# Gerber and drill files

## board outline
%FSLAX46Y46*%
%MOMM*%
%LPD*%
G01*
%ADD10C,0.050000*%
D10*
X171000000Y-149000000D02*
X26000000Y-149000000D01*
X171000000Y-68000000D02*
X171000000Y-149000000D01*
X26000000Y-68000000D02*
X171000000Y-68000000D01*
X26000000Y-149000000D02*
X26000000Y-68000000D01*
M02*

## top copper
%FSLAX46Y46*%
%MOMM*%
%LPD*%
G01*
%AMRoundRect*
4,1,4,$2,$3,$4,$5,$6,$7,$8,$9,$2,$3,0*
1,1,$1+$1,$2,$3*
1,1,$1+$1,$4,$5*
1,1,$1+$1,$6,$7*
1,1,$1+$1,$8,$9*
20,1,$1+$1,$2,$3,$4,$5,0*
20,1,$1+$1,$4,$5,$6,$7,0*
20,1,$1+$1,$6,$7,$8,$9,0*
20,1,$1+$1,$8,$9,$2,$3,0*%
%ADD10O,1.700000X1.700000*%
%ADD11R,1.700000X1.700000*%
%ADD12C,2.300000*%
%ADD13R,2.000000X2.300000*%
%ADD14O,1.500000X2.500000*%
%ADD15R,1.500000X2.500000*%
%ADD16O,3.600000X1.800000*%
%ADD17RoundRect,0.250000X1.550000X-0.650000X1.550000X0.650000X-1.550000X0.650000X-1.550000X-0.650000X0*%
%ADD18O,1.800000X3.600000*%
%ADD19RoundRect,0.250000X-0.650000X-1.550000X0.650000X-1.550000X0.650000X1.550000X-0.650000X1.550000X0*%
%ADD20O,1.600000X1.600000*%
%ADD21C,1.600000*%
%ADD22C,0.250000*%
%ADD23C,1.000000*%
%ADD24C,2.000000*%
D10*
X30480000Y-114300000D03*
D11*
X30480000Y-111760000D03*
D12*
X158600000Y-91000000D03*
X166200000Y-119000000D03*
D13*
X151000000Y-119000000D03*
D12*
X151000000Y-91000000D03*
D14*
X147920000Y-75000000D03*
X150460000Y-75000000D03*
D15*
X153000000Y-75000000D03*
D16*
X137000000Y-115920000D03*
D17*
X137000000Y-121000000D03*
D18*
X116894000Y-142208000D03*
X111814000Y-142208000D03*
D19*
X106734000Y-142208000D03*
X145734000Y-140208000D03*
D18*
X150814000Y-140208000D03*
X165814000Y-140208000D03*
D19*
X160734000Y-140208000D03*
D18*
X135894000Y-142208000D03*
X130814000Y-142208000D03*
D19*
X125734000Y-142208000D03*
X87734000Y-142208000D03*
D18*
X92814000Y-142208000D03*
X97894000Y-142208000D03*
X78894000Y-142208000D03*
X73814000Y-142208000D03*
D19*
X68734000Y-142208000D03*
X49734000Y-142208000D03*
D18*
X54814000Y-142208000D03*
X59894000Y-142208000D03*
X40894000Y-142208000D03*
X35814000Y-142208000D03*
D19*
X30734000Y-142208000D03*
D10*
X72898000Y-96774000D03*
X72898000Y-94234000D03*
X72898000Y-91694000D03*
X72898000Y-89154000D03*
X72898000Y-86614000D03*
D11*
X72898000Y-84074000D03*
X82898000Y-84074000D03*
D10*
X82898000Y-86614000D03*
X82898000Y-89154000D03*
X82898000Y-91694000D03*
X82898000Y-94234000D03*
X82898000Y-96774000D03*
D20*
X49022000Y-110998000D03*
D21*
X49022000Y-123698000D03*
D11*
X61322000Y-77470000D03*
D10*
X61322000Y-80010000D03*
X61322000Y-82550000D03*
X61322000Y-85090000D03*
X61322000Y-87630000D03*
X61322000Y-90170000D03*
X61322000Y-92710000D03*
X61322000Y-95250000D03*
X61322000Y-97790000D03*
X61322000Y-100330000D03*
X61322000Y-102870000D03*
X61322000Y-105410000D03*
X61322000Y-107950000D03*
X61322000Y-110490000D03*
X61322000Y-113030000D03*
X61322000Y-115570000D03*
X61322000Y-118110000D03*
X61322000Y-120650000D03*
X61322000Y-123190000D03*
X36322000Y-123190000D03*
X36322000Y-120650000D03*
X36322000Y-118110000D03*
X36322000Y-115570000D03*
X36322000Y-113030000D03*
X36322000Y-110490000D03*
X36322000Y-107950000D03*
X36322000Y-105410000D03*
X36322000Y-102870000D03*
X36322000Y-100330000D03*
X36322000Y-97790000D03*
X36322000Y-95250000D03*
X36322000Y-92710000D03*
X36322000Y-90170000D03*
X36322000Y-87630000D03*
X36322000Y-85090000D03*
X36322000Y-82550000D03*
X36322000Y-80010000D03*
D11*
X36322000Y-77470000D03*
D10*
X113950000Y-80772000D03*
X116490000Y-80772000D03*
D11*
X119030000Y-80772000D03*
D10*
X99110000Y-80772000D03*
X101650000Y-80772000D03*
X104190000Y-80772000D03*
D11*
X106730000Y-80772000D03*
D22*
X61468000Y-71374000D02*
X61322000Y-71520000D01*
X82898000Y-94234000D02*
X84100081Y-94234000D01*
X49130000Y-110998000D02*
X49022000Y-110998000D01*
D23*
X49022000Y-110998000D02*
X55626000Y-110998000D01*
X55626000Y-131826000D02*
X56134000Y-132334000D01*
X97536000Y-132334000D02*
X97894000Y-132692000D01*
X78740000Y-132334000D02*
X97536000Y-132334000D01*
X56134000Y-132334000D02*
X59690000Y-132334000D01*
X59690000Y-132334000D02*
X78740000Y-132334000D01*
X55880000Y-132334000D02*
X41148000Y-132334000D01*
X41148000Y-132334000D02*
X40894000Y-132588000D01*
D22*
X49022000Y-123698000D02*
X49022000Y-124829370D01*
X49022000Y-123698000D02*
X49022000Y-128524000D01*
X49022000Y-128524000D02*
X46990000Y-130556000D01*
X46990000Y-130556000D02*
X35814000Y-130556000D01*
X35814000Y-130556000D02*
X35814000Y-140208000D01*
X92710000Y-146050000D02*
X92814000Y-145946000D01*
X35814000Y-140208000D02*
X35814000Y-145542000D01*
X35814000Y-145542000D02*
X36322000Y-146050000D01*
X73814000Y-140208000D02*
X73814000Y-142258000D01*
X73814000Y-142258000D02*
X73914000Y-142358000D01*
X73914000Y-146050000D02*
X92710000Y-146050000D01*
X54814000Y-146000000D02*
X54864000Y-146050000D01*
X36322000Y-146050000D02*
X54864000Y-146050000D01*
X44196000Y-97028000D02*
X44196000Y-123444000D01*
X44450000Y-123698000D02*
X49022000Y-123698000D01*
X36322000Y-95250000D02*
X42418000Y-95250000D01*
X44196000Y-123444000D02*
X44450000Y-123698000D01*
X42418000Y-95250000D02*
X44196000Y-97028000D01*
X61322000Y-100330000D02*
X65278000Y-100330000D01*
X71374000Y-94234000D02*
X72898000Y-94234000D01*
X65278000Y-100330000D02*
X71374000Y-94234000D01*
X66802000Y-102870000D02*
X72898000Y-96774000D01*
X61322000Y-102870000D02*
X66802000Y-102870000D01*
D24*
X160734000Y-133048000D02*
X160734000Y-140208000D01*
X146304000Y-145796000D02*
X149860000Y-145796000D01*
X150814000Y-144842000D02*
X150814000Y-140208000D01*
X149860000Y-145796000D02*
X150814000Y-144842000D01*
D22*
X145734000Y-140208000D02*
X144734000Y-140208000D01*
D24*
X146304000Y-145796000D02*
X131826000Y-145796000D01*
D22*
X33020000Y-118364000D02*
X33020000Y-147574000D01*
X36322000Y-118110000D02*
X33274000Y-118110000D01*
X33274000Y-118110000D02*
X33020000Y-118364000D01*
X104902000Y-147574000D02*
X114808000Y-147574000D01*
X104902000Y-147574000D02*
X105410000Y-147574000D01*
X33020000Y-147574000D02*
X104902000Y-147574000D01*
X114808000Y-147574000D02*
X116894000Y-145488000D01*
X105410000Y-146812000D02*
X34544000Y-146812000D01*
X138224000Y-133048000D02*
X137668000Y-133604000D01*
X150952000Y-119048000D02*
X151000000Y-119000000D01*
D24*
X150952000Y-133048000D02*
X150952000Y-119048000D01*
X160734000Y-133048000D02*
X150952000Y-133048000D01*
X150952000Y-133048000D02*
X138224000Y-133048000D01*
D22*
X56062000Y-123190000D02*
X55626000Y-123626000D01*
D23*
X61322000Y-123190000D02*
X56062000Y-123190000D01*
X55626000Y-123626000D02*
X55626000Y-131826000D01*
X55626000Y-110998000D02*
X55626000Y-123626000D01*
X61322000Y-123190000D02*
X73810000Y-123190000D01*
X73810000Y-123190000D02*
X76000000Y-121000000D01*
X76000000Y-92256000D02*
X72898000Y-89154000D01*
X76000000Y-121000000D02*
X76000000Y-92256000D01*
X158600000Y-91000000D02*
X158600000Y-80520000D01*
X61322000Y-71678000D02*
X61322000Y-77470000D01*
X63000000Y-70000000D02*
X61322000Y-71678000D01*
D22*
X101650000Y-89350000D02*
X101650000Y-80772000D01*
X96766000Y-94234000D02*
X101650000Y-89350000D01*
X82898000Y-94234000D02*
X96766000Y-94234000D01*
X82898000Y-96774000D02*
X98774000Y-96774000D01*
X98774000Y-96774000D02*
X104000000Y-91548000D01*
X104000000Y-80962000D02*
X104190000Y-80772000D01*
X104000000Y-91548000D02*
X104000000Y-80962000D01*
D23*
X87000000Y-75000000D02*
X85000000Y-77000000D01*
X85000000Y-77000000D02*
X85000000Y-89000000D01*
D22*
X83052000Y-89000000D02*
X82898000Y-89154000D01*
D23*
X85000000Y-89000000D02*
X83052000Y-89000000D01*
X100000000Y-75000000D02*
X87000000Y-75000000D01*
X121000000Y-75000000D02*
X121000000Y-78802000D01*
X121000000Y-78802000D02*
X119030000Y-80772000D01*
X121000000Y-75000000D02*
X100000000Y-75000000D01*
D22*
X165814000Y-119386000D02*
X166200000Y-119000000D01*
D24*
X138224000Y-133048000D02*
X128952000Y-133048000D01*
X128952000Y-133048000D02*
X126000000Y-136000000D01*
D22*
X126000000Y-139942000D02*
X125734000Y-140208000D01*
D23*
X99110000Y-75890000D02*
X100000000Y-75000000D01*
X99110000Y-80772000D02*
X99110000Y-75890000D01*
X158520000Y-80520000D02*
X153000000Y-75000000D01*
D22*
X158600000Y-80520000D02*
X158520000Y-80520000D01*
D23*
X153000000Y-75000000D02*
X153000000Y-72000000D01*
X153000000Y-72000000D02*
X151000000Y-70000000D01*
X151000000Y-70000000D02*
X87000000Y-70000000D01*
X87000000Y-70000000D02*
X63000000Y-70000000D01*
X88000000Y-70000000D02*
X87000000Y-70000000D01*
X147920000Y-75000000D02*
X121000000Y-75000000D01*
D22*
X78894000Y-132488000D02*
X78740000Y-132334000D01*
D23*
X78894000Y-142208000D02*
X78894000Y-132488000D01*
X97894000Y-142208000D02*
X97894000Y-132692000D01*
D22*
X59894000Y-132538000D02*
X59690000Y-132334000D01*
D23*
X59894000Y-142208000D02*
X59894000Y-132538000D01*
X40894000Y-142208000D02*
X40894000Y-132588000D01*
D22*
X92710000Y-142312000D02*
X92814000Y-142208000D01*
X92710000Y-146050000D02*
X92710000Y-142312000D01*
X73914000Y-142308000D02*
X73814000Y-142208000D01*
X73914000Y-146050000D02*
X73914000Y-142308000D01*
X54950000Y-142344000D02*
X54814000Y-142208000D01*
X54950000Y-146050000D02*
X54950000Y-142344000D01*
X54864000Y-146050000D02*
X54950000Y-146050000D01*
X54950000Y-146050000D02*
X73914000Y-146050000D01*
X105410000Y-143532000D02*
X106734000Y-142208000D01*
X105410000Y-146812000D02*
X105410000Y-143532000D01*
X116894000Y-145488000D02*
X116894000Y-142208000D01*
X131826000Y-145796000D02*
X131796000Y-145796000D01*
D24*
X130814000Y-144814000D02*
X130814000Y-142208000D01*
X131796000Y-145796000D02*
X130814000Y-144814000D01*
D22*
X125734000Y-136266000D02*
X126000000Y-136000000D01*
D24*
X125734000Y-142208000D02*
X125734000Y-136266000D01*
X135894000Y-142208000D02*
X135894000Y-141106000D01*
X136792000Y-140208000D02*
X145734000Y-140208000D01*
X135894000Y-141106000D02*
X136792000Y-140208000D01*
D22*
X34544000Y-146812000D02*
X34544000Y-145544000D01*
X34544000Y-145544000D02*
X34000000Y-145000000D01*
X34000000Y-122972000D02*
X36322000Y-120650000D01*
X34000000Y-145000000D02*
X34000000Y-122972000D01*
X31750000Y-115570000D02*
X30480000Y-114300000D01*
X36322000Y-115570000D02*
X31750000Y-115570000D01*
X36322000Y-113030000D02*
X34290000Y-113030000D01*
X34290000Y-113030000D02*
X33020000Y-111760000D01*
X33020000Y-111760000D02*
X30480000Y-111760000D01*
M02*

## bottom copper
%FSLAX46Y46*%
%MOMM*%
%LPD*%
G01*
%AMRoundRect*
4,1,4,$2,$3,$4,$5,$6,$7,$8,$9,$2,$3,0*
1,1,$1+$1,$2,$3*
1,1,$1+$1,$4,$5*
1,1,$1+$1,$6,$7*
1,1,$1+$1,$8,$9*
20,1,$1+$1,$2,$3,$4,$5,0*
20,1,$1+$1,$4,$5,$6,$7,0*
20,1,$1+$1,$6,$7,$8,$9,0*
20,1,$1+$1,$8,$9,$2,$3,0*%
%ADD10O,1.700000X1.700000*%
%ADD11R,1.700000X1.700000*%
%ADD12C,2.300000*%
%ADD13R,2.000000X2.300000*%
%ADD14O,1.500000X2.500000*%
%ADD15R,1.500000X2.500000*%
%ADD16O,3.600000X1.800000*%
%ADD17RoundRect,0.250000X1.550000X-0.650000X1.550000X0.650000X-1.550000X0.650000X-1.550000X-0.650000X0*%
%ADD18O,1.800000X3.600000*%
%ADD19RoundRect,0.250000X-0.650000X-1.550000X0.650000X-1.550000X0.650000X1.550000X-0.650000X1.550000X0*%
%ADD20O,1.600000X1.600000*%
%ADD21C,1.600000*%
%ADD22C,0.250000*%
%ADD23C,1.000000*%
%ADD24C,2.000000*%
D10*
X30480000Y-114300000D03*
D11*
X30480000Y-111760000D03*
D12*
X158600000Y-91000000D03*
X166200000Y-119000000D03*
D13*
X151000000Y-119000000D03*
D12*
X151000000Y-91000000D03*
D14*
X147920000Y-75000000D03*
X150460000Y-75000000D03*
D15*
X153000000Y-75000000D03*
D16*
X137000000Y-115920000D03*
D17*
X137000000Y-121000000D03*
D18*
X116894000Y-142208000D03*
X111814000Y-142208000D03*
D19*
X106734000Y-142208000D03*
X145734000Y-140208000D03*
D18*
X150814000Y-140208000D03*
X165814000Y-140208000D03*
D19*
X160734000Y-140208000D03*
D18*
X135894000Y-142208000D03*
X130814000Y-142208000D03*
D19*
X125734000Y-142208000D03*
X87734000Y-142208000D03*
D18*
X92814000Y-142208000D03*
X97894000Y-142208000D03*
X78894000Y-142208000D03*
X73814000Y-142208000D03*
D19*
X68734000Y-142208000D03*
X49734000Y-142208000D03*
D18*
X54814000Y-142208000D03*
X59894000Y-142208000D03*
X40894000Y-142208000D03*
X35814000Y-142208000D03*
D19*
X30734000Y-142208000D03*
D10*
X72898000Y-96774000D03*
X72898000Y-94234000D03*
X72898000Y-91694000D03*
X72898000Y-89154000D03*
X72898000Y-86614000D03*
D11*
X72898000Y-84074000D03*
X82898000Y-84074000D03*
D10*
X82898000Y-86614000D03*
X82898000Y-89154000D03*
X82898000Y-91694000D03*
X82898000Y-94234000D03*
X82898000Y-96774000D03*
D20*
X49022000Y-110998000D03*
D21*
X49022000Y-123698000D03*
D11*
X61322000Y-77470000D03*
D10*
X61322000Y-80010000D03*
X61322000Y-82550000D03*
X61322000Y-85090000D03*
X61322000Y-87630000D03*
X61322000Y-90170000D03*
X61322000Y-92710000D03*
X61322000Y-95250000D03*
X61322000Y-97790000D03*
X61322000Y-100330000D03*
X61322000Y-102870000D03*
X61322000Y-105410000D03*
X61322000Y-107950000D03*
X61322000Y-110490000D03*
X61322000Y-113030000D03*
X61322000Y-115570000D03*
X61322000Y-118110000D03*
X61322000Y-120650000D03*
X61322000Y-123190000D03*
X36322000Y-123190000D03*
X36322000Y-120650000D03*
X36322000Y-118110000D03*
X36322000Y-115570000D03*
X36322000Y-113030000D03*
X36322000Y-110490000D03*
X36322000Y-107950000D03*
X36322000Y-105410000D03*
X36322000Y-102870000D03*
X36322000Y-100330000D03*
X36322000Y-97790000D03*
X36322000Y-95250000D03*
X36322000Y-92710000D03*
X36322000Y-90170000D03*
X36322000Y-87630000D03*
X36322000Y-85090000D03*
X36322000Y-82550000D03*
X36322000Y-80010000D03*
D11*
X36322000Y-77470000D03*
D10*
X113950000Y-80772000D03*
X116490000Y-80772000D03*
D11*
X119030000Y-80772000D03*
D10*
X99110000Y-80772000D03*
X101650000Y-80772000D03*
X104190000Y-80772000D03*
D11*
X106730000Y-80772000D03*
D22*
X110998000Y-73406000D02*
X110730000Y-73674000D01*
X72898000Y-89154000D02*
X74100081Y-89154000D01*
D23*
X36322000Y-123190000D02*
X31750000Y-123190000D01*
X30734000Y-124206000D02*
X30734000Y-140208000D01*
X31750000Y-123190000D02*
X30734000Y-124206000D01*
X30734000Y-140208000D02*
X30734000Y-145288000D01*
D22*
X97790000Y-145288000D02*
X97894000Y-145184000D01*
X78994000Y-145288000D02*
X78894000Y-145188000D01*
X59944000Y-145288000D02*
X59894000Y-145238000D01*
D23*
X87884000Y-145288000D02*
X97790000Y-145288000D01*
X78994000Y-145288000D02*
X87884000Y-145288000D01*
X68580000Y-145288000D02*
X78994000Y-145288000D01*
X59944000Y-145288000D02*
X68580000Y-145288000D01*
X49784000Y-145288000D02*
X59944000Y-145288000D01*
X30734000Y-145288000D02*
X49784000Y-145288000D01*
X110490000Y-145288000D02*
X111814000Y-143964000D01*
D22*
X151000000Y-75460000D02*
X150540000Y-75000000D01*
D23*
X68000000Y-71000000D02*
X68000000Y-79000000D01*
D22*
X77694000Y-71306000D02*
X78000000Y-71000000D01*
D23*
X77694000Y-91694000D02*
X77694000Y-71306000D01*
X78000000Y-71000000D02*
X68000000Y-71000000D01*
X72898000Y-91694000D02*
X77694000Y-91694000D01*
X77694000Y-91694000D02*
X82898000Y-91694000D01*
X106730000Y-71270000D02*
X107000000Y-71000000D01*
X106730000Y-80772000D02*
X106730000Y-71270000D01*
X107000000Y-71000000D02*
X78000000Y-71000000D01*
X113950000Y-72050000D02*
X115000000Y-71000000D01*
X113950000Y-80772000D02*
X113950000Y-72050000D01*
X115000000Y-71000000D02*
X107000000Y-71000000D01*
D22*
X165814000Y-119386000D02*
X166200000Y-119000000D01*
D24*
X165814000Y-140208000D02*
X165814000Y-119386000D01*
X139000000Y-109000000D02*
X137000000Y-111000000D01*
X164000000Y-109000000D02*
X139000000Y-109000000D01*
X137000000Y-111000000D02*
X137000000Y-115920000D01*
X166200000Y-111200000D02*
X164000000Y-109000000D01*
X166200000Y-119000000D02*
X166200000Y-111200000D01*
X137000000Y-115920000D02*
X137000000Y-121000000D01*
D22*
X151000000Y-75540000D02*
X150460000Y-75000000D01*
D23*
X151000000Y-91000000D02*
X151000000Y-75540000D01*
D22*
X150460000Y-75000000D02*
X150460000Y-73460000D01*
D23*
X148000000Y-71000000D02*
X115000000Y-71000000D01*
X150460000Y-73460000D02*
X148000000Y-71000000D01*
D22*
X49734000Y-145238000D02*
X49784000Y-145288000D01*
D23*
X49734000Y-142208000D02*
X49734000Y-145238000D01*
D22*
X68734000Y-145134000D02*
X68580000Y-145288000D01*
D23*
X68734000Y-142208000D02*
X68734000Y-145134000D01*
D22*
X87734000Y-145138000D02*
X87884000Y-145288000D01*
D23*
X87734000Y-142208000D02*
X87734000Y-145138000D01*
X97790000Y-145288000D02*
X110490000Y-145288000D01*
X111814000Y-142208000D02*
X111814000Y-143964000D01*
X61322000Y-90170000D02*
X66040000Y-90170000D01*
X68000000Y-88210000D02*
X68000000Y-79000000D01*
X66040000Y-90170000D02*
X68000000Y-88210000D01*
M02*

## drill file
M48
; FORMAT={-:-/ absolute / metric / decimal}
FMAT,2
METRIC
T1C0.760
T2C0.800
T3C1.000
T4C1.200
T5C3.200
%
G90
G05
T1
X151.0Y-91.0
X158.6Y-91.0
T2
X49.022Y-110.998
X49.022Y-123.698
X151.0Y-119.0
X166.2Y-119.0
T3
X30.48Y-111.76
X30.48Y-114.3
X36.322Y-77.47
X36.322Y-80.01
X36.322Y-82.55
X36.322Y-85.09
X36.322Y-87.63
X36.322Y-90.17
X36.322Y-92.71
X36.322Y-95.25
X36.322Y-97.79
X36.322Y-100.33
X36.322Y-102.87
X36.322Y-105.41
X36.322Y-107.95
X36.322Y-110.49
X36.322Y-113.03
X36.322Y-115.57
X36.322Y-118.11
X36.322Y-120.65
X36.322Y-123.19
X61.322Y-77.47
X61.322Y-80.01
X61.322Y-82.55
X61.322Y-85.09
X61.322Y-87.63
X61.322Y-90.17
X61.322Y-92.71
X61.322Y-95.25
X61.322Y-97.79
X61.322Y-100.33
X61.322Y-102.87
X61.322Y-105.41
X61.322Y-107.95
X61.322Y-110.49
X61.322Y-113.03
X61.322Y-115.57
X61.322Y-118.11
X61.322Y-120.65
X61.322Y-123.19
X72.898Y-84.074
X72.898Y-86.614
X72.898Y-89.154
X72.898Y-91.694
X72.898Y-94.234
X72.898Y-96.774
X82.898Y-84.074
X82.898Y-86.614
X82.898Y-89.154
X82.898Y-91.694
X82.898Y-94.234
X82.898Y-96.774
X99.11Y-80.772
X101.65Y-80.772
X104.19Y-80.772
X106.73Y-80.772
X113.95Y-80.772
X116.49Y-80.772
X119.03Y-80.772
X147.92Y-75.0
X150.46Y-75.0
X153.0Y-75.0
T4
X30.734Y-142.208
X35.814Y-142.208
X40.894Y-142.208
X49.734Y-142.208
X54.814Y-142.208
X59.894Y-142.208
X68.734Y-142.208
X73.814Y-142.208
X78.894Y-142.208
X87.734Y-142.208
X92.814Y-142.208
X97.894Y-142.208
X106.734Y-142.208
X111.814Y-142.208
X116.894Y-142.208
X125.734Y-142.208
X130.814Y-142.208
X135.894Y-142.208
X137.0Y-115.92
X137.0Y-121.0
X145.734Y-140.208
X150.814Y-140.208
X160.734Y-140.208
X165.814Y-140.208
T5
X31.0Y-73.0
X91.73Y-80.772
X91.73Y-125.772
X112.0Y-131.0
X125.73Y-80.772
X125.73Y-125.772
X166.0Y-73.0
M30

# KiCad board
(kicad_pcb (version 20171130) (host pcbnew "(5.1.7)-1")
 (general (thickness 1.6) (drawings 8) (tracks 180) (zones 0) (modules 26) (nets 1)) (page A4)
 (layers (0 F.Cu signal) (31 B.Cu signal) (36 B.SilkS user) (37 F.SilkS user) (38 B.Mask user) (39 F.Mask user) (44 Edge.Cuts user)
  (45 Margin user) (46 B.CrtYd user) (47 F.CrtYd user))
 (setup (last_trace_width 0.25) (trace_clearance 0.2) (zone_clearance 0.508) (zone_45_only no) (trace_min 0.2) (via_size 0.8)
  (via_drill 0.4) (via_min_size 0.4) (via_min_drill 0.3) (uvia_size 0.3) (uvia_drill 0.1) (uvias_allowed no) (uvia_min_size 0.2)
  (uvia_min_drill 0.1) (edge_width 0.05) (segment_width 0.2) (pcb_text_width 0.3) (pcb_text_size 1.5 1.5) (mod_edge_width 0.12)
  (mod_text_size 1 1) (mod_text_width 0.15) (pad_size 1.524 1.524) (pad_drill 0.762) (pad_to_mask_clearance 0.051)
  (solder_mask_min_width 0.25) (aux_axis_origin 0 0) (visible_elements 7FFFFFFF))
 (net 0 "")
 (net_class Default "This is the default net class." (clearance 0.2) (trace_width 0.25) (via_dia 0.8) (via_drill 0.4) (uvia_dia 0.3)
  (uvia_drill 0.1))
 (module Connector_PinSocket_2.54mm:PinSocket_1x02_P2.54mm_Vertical (layer F.Cu) (at 30.48 111.76)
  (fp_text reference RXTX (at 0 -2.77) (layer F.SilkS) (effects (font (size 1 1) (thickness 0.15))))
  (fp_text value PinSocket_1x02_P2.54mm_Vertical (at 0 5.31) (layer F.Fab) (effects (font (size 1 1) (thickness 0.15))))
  (pad 2 thru_hole oval (at 0 2.54) (size 1.7 1.7) (drill 1) (layers *.Cu *.Mask))
  (pad 1 thru_hole rect (at 0 0) (size 1.7 1.7) (drill 1) (layers *.Cu *.Mask)))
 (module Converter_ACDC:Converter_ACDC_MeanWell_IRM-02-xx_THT (layer F.Cu) (at 151 119 90)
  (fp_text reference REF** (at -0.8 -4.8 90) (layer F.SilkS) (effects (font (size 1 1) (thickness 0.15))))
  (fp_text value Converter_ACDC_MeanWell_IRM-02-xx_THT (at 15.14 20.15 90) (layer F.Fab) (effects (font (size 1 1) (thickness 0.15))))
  (pad 4 thru_hole circle (at 28 7.6 90) (size 2.3 2.3) (drill 0.76) (layers *.Cu *.Mask))
  (pad 2 thru_hole circle (at 0 15.2 90) (size 2.3 2.3) (drill 0.8) (layers *.Cu *.Mask))
  (pad 1 thru_hole rect (at 0 0 90) (size 2.3 2) (drill 0.8) (layers *.Cu *.Mask))
  (pad 3 thru_hole circle (at 28 0 90) (size 2.3 2.3) (drill 0.76) (layers *.Cu *.Mask)))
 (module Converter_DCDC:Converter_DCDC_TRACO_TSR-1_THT (layer F.Cu) (at 153 75 180)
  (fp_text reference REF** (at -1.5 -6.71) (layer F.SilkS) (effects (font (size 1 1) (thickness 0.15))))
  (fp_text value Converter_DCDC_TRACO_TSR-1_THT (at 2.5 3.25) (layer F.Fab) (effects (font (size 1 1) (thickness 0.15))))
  (pad 3 thru_hole oval (at 5.08 0 180) (size 1.5 2.5) (drill 1) (layers *.Cu *.Mask))
  (pad 2 thru_hole oval (at 2.54 0 180) (size 1.5 2.5) (drill 1) (layers *.Cu *.Mask))
  (pad 1 thru_hole rect (at 0 0 180) (size 1.5 2.5) (drill 1) (layers *.Cu *.Mask)))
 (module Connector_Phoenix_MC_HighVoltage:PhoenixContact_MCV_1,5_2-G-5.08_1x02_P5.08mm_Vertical (layer F.Cu) (at 137 121 90)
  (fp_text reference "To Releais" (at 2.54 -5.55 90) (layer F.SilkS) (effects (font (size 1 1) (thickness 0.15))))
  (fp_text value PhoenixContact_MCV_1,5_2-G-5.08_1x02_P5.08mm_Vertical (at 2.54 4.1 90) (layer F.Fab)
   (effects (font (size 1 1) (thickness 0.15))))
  (pad 2 thru_hole oval (at 5.08 0 90) (size 1.8 3.6) (drill 1.2) (layers *.Cu *.Mask))
  (pad 1 thru_hole roundrect (at 0 0 90) (size 1.8 3.6) (drill 1.2) (layers *.Cu *.Mask) (roundrect_rratio 0.138889)))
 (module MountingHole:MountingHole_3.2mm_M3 (layer F.Cu) (at 112 131)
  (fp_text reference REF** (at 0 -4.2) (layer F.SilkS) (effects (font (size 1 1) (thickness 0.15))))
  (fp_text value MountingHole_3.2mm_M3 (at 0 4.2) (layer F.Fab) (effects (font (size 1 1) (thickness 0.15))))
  (pad 1 np_thru_hole circle (at 0 0) (size 3.2 3.2) (drill 3.2) (layers *.Cu *.Mask)))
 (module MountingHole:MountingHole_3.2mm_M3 (layer F.Cu) (at 166 73)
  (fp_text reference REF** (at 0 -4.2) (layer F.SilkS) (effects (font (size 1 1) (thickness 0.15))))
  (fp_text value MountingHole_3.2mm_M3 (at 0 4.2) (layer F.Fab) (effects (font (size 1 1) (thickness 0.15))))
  (pad 1 np_thru_hole circle (at 0 0) (size 3.2 3.2) (drill 3.2) (layers *.Cu *.Mask)))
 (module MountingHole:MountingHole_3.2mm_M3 (layer F.Cu) (at 31 73)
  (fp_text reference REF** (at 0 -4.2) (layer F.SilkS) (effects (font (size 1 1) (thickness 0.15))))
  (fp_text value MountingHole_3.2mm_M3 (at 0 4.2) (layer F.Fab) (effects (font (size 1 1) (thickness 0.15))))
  (pad 1 np_thru_hole circle (at 0 0) (size 3.2 3.2) (drill 3.2) (layers *.Cu *.Mask)))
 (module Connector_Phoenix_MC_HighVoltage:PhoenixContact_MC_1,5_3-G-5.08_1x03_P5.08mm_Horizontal (layer F.Cu) (at 106.734 142.208)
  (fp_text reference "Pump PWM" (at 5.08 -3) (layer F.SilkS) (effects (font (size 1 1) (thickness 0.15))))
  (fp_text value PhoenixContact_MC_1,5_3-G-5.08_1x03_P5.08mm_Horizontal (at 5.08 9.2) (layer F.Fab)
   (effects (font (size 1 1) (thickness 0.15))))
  (pad 3 thru_hole oval (at 10.16 0) (size 1.8 3.6) (drill 1.2) (layers *.Cu *.Mask))
  (pad 2 thru_hole oval (at 5.08 0) (size 1.8 3.6) (drill 1.2) (layers *.Cu *.Mask))
  (pad 1 thru_hole roundrect (at 0 0) (size 1.8 3.6) (drill 1.2) (layers *.Cu *.Mask) (roundrect_rratio 0.138889)))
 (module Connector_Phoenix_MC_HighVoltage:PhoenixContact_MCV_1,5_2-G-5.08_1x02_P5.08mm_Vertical (layer F.Cu) (at 145.734 140.208)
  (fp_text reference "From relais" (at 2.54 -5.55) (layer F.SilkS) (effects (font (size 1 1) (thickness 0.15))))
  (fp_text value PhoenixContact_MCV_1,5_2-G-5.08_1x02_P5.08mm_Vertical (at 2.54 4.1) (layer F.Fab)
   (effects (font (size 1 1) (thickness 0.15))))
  (pad 1 thru_hole roundrect (at 0 0) (size 1.8 3.6) (drill 1.2) (layers *.Cu *.Mask) (roundrect_rratio 0.138889))
  (pad 2 thru_hole oval (at 5.08 0) (size 1.8 3.6) (drill 1.2) (layers *.Cu *.Mask)))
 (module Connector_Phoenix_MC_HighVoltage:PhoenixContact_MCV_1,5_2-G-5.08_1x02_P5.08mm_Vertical (layer F.Cu) (at 160.734 140.208)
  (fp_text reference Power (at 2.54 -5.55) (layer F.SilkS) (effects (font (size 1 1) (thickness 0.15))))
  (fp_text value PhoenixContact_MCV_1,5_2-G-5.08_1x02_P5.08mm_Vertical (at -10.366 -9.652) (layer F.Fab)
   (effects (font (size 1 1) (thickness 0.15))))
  (pad 2 thru_hole oval (at 5.08 0) (size 1.8 3.6) (drill 1.2) (layers *.Cu *.Mask))
  (pad 1 thru_hole roundrect (at 0 0) (size 1.8 3.6) (drill 1.2) (layers *.Cu *.Mask) (roundrect_rratio 0.138889)))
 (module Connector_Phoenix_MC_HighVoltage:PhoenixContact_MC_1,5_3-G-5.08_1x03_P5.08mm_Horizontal (layer F.Cu) (at 125.734 142.208)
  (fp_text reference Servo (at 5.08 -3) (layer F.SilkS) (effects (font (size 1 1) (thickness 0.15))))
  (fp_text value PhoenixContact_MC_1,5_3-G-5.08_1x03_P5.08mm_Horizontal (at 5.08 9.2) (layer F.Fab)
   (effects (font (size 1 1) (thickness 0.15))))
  (pad 3 thru_hole oval (at 10.16 0) (size 1.8 3.6) (drill 1.2) (layers *.Cu *.Mask))
  (pad 2 thru_hole oval (at 5.08 0) (size 1.8 3.6) (drill 1.2) (layers *.Cu *.Mask))
  (pad 1 thru_hole roundrect (at 0 0) (size 1.8 3.6) (drill 1.2) (layers *.Cu *.Mask) (roundrect_rratio 0.138889)))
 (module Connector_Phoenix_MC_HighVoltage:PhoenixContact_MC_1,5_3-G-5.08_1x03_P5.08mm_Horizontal (layer F.Cu) (at 87.734 142.208)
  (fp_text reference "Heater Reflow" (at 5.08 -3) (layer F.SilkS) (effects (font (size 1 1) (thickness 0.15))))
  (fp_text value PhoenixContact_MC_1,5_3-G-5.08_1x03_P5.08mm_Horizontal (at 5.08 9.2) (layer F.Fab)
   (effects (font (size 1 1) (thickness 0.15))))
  (pad 1 thru_hole roundrect (at 0 0) (size 1.8 3.6) (drill 1.2) (layers *.Cu *.Mask) (roundrect_rratio 0.138889))
  (pad 2 thru_hole oval (at 5.08 0) (size 1.8 3.6) (drill 1.2) (layers *.Cu *.Mask))
  (pad 3 thru_hole oval (at 10.16 0) (size 1.8 3.6) (drill 1.2) (layers *.Cu *.Mask)))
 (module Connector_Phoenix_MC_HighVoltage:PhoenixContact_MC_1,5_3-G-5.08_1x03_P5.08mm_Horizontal (layer F.Cu) (at 68.734 142.208)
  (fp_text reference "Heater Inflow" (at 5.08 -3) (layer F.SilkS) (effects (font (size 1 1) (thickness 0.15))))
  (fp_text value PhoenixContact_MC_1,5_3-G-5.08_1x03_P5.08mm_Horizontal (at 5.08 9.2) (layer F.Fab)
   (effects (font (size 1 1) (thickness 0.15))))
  (pad 3 thru_hole oval (at 10.16 0) (size 1.8 3.6) (drill 1.2) (layers *.Cu *.Mask))
  (pad 2 thru_hole oval (at 5.08 0) (size 1.8 3.6) (drill 1.2) (layers *.Cu *.Mask))
  (pad 1 thru_hole roundrect (at 0 0) (size 1.8 3.6) (drill 1.2) (layers *.Cu *.Mask) (roundrect_rratio 0.138889)))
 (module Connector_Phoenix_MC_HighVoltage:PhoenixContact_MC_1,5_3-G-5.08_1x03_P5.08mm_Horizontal (layer F.Cu) (at 49.734 142.208)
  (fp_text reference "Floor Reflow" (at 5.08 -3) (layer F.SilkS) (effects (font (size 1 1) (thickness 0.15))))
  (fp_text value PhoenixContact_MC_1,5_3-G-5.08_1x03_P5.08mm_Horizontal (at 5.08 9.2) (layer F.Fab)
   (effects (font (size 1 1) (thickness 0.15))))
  (pad 1 thru_hole roundrect (at 0 0) (size 1.8 3.6) (drill 1.2) (layers *.Cu *.Mask) (roundrect_rratio 0.138889))
  (pad 2 thru_hole oval (at 5.08 0) (size 1.8 3.6) (drill 1.2) (layers *.Cu *.Mask))
  (pad 3 thru_hole oval (at 10.16 0) (size 1.8 3.6) (drill 1.2) (layers *.Cu *.Mask)))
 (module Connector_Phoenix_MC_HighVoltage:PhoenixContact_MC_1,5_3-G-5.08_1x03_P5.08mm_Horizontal (layer F.Cu) (at 30.734 142.208)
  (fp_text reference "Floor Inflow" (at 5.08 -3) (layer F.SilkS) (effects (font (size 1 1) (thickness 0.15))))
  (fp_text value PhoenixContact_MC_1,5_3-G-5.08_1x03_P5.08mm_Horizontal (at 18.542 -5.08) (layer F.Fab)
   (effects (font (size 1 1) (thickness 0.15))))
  (pad 3 thru_hole oval (at 10.16 0) (size 1.8 3.6) (drill 1.2) (layers *.Cu *.Mask))
  (pad 2 thru_hole oval (at 5.08 0) (size 1.8 3.6) (drill 1.2) (layers *.Cu *.Mask))
  (pad 1 thru_hole roundrect (at 0 0) (size 1.8 3.6) (drill 1.2) (layers *.Cu *.Mask) (roundrect_rratio 0.138889)))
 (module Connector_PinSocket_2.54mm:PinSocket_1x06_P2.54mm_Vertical (layer F.Cu) (at 72.898 84.074)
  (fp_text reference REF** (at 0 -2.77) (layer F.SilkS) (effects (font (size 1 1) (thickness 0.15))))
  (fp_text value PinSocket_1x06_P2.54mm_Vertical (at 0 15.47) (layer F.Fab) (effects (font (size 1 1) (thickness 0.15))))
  (pad 6 thru_hole oval (at 0 12.7) (size 1.7 1.7) (drill 1) (layers *.Cu *.Mask))
  (pad 5 thru_hole oval (at 0 10.16) (size 1.7 1.7) (drill 1) (layers *.Cu *.Mask))
  (pad 4 thru_hole oval (at 0 7.62) (size 1.7 1.7) (drill 1) (layers *.Cu *.Mask))
  (pad 3 thru_hole oval (at 0 5.08) (size 1.7 1.7) (drill 1) (layers *.Cu *.Mask))
  (pad 2 thru_hole oval (at 0 2.54) (size 1.7 1.7) (drill 1) (layers *.Cu *.Mask))
  (pad 1 thru_hole rect (at 0 0) (size 1.7 1.7) (drill 1) (layers *.Cu *.Mask)))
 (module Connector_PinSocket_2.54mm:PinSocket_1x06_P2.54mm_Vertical (layer F.Cu) (at 82.898 84.074)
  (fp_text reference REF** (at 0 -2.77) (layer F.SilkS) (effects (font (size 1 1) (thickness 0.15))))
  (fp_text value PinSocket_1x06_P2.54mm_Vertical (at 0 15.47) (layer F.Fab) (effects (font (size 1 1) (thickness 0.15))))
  (pad 1 thru_hole rect (at 0 0) (size 1.7 1.7) (drill 1) (layers *.Cu *.Mask))
  (pad 2 thru_hole oval (at 0 2.54) (size 1.7 1.7) (drill 1) (layers *.Cu *.Mask))
  (pad 3 thru_hole oval (at 0 5.08) (size 1.7 1.7) (drill 1) (layers *.Cu *.Mask))
  (pad 4 thru_hole oval (at 0 7.62) (size 1.7 1.7) (drill 1) (layers *.Cu *.Mask))
  (pad 5 thru_hole oval (at 0 10.16) (size 1.7 1.7) (drill 1) (layers *.Cu *.Mask))
  (pad 6 thru_hole oval (at 0 12.7) (size 1.7 1.7) (drill 1) (layers *.Cu *.Mask)))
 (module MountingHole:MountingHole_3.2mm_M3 (layer F.Cu) (at 125.73 125.772)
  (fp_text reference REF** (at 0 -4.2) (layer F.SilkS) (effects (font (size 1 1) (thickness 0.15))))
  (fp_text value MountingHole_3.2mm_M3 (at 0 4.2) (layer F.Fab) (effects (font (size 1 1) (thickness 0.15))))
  (pad 1 np_thru_hole circle (at 0 0) (size 3.2 3.2) (drill 3.2) (layers *.Cu *.Mask)))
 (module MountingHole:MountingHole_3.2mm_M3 (layer F.Cu) (at 91.73 125.772)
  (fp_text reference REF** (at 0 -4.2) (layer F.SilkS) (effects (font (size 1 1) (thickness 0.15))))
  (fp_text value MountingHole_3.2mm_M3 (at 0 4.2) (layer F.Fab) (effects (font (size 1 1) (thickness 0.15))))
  (pad 1 np_thru_hole circle (at 0 0) (size 3.2 3.2) (drill 3.2) (layers *.Cu *.Mask)))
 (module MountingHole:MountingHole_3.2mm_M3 (layer F.Cu) (at 125.73 80.772)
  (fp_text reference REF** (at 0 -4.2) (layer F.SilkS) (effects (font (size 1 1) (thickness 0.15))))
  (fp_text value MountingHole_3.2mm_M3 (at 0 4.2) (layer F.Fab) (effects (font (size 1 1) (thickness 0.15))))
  (pad 1 np_thru_hole circle (at 0 0) (size 3.2 3.2) (drill 3.2) (layers *.Cu *.Mask)))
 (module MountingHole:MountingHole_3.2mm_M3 (layer F.Cu) (at 91.73 80.772)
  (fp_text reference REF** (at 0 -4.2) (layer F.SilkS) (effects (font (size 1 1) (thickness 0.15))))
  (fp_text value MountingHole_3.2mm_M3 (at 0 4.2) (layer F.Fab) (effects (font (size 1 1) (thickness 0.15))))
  (pad 1 np_thru_hole circle (at 0 0) (size 3.2 3.2) (drill 3.2) (layers *.Cu *.Mask)))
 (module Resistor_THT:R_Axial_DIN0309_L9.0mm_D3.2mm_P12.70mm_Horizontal (layer F.Cu) (at 49.022 123.698 90)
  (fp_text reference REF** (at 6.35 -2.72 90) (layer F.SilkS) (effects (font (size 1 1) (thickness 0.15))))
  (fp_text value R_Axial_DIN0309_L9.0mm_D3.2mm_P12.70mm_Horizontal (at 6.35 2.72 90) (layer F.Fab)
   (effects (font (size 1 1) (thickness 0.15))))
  (pad 2 thru_hole oval (at 12.7 0 90) (size 1.6 1.6) (drill 0.8) (layers *.Cu *.Mask))
  (pad 1 thru_hole circle (at 0 0 90) (size 1.6 1.6) (drill 0.8) (layers *.Cu *.Mask)))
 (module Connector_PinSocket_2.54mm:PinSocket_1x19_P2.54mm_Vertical (layer F.Cu) (at 61.322 77.47)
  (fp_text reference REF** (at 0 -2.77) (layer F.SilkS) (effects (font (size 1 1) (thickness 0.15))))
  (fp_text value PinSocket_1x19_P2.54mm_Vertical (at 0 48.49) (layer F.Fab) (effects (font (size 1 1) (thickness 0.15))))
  (pad 1 thru_hole rect (at 0 0) (size 1.7 1.7) (drill 1) (layers *.Cu *.Mask))
  (pad 2 thru_hole oval (at 0 2.54) (size 1.7 1.7) (drill 1) (layers *.Cu *.Mask))
  (pad 3 thru_hole oval (at 0 5.08) (size 1.7 1.7) (drill 1) (layers *.Cu *.Mask))
  (pad 4 thru_hole oval (at 0 7.62) (size 1.7 1.7) (drill 1) (layers *.Cu *.Mask))
  (pad 5 thru_hole oval (at 0 10.16) (size 1.7 1.7) (drill 1) (layers *.Cu *.Mask))
  (pad 6 thru_hole oval (at 0 12.7) (size 1.7 1.7) (drill 1) (layers *.Cu *.Mask))
  (pad 7 thru_hole oval (at 0 15.24) (size 1.7 1.7) (drill 1) (layers *.Cu *.Mask))
  (pad 8 thru_hole oval (at 0 17.78) (size 1.7 1.7) (drill 1) (layers *.Cu *.Mask))
  (pad 9 thru_hole oval (at 0 20.32) (size 1.7 1.7) (drill 1) (layers *.Cu *.Mask))
  (pad 10 thru_hole oval (at 0 22.86) (size 1.7 1.7) (drill 1) (layers *.Cu *.Mask))
  (pad 11 thru_hole oval (at 0 25.4) (size 1.7 1.7) (drill 1) (layers *.Cu *.Mask))
  (pad 12 thru_hole oval (at 0 27.94) (size 1.7 1.7) (drill 1) (layers *.Cu *.Mask))
  (pad 13 thru_hole oval (at 0 30.48) (size 1.7 1.7) (drill 1) (layers *.Cu *.Mask))
  (pad 14 thru_hole oval (at 0 33.02) (size 1.7 1.7) (drill 1) (layers *.Cu *.Mask))
  (pad 15 thru_hole oval (at 0 35.56) (size 1.7 1.7) (drill 1) (layers *.Cu *.Mask))
  (pad 16 thru_hole oval (at 0 38.1) (size 1.7 1.7) (drill 1) (layers *.Cu *.Mask))
  (pad 17 thru_hole oval (at 0 40.64) (size 1.7 1.7) (drill 1) (layers *.Cu *.Mask))
  (pad 18 thru_hole oval (at 0 43.18) (size 1.7 1.7) (drill 1) (layers *.Cu *.Mask))
  (pad 19 thru_hole oval (at 0 45.72) (size 1.7 1.7) (drill 1) (layers *.Cu *.Mask)))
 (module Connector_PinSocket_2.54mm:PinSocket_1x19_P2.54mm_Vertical (layer F.Cu) (at 36.322 77.47)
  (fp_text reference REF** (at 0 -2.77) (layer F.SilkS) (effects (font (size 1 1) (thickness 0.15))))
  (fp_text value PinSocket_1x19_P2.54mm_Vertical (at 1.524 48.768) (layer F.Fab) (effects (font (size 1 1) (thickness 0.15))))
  (pad 19 thru_hole oval (at 0 45.72) (size 1.7 1.7) (drill 1) (layers *.Cu *.Mask))
  (pad 18 thru_hole oval (at 0 43.18) (size 1.7 1.7) (drill 1) (layers *.Cu *.Mask))
  (pad 17 thru_hole oval (at 0 40.64) (size 1.7 1.7) (drill 1) (layers *.Cu *.Mask))
  (pad 16 thru_hole oval (at 0 38.1) (size 1.7 1.7) (drill 1) (layers *.Cu *.Mask))
  (pad 15 thru_hole oval (at 0 35.56) (size 1.7 1.7) (drill 1) (layers *.Cu *.Mask))
  (pad 14 thru_hole oval (at 0 33.02) (size 1.7 1.7) (drill 1) (layers *.Cu *.Mask))
  (pad 13 thru_hole oval (at 0 30.48) (size 1.7 1.7) (drill 1) (layers *.Cu *.Mask))
  (pad 12 thru_hole oval (at 0 27.94) (size 1.7 1.7) (drill 1) (layers *.Cu *.Mask))
  (pad 11 thru_hole oval (at 0 25.4) (size 1.7 1.7) (drill 1) (layers *.Cu *.Mask))
  (pad 10 thru_hole oval (at 0 22.86) (size 1.7 1.7) (drill 1) (layers *.Cu *.Mask))
  (pad 9 thru_hole oval (at 0 20.32) (size 1.7 1.7) (drill 1) (layers *.Cu *.Mask))
  (pad 8 thru_hole oval (at 0 17.78) (size 1.7 1.7) (drill 1) (layers *.Cu *.Mask))
  (pad 7 thru_hole oval (at 0 15.24) (size 1.7 1.7) (drill 1) (layers *.Cu *.Mask))
  (pad 6 thru_hole oval (at 0 12.7) (size 1.7 1.7) (drill 1) (layers *.Cu *.Mask))
  (pad 5 thru_hole oval (at 0 10.16) (size 1.7 1.7) (drill 1) (layers *.Cu *.Mask))
  (pad 4 thru_hole oval (at 0 7.62) (size 1.7 1.7) (drill 1) (layers *.Cu *.Mask))
  (pad 3 thru_hole oval (at 0 5.08) (size 1.7 1.7) (drill 1) (layers *.Cu *.Mask))
  (pad 2 thru_hole oval (at 0 2.54) (size 1.7 1.7) (drill 1) (layers *.Cu *.Mask))
  (pad 1 thru_hole rect (at 0 0) (size 1.7 1.7) (drill 1) (layers *.Cu *.Mask)))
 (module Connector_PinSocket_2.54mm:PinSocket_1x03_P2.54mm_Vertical (layer F.Cu) (at 119.03 80.772 270)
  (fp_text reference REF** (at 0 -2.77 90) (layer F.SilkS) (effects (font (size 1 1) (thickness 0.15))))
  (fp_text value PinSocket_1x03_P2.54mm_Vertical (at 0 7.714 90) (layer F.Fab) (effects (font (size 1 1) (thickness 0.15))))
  (pad 3 thru_hole oval (at 0 5.08 270) (size 1.7 1.7) (drill 1) (layers *.Cu *.Mask))
  (pad 2 thru_hole oval (at 0 2.54 270) (size 1.7 1.7) (drill 1) (layers *.Cu *.Mask))
  (pad 1 thru_hole rect (at 0 0 270) (size 1.7 1.7) (drill 1) (layers *.Cu *.Mask)))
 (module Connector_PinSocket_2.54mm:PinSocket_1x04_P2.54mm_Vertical (layer F.Cu) (at 106.73 80.772 270)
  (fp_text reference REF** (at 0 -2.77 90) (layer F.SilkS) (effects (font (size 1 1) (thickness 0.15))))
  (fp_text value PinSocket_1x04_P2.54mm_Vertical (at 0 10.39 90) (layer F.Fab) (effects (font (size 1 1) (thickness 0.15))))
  (pad 4 thru_hole oval (at 0 7.62 270) (size 1.7 1.7) (drill 1) (layers *.Cu *.Mask))
  (pad 3 thru_hole oval (at 0 5.08 270) (size 1.7 1.7) (drill 1) (layers *.Cu *.Mask))
  (pad 2 thru_hole oval (at 0 2.54 270) (size 1.7 1.7) (drill 1) (layers *.Cu *.Mask))
  (pad 1 thru_hole rect (at 0 0 270) (size 1.7 1.7) (drill 1) (layers *.Cu *.Mask)))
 (gr_line (start 171 149) (end 26 149) (layer Edge.Cuts) (width 0.05))
 (gr_line (start 171 68) (end 171 149) (layer Edge.Cuts) (width 0.05))
 (gr_line (start 26 68) (end 171 68) (layer Edge.Cuts) (width 0.05))
 (gr_line (start 26 149) (end 26 68) (layer Edge.Cuts) (width 0.05))
 (segment (start 61.468 71.374) (end 61.322 71.52) (width 0.25) (layer F.Cu) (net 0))
 (segment (start 82.898 94.234) (end 84.100081 94.234) (width 0.25) (layer F.Cu) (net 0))
 (segment (start 49.13 110.998) (end 49.022 110.998) (width 0.25) (layer F.Cu) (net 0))
 (segment (start 49.022 110.998) (end 55.626 110.998) (width 1) (layer F.Cu) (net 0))
 (segment (start 55.626 131.826) (end 56.134 132.334) (width 1) (layer F.Cu) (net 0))
 (segment (start 97.536 132.334) (end 97.894 132.692) (width 1) (layer F.Cu) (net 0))
 (segment (start 78.74 132.334) (end 97.536 132.334) (width 1) (layer F.Cu) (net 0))
 (segment (start 56.134 132.334) (end 59.69 132.334) (width 1) (layer F.Cu) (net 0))
 (segment (start 59.69 132.334) (end 78.74 132.334) (width 1) (layer F.Cu) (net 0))
 (segment (start 55.88 132.334) (end 41.148 132.334) (width 1) (layer F.Cu) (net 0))
 (segment (start 41.148 132.334) (end 40.894 132.588) (width 1) (layer F.Cu) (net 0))
 (segment (start 49.022 123.698) (end 49.022 124.82937) (width 0.25) (layer F.Cu) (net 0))
 (segment (start 49.022 123.698) (end 49.022 128.524) (width 0.25) (layer F.Cu) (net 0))
 (segment (start 49.022 128.524) (end 46.99 130.556) (width 0.25) (layer F.Cu) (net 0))
 (segment (start 46.99 130.556) (end 35.814 130.556) (width 0.25) (layer F.Cu) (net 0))
 (segment (start 35.814 130.556) (end 35.814 140.208) (width 0.25) (layer F.Cu) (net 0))
 (segment (start 92.71 146.05) (end 92.814 145.946) (width 0.25) (layer F.Cu) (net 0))
 (segment (start 35.814 140.208) (end 35.814 145.542) (width 0.25) (layer F.Cu) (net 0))
 (segment (start 35.814 145.542) (end 36.322 146.05) (width 0.25) (layer F.Cu) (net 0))
 (segment (start 73.814 140.208) (end 73.814 142.258) (width 0.25) (layer F.Cu) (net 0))
 (segment (start 73.814 142.258) (end 73.914 142.358) (width 0.25) (layer F.Cu) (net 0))
 (segment (start 73.914 146.05) (end 92.71 146.05) (width 0.25) (layer F.Cu) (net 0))
 (segment (start 54.814 146) (end 54.864 146.05) (width 0.25) (layer F.Cu) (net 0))
 (segment (start 36.322 146.05) (end 54.864 146.05) (width 0.25) (layer F.Cu) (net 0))
 (segment (start 44.196 97.028) (end 44.196 123.444) (width 0.25) (layer F.Cu) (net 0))
 (segment (start 44.45 123.698) (end 49.022 123.698) (width 0.25) (layer F.Cu) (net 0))
 (segment (start 36.322 95.25) (end 42.418 95.25) (width 0.25) (layer F.Cu) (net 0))
 (segment (start 44.196 123.444) (end 44.45 123.698) (width 0.25) (layer F.Cu) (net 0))
 (segment (start 42.418 95.25) (end 44.196 97.028) (width 0.25) (layer F.Cu) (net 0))
 (segment (start 61.322 100.33) (end 65.278 100.33) (width 0.25) (layer F.Cu) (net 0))
 (segment (start 71.374 94.234) (end 72.898 94.234) (width 0.25) (layer F.Cu) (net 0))
 (segment (start 65.278 100.33) (end 71.374 94.234) (width 0.25) (layer F.Cu) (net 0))
 (segment (start 66.802 102.87) (end 72.898 96.774) (width 0.25) (layer F.Cu) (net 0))
 (segment (start 61.322 102.87) (end 66.802 102.87) (width 0.25) (layer F.Cu) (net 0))
 (segment (start 160.734 133.048) (end 160.734 140.208) (width 2) (layer F.Cu) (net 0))
 (segment (start 110.998 73.406) (end 110.73 73.674) (width 0.25) (layer B.Cu) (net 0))
 (segment (start 72.898 89.154) (end 74.100081 89.154) (width 0.25) (layer B.Cu) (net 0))
 (segment (start 36.322 123.19) (end 31.75 123.19) (width 1) (layer B.Cu) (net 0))
 (segment (start 30.734 124.206) (end 30.734 140.208) (width 1) (layer B.Cu) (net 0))
 (segment (start 31.75 123.19) (end 30.734 124.206) (width 1) (layer B.Cu) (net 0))
 (segment (start 30.734 140.208) (end 30.734 145.288) (width 1) (layer B.Cu) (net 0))
 (segment (start 97.79 145.288) (end 97.894 145.184) (width 0.25) (layer B.Cu) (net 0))
 (segment (start 78.994 145.288) (end 78.894 145.188) (width 0.25) (layer B.Cu) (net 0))
 (segment (start 59.944 145.288) (end 59.894 145.238) (width 0.25) (layer B.Cu) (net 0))
 (segment (start 87.884 145.288) (end 97.79 145.288) (width 1) (layer B.Cu) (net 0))
 (segment (start 78.994 145.288) (end 87.884 145.288) (width 1) (layer B.Cu) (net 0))
 (segment (start 68.58 145.288) (end 78.994 145.288) (width 1) (layer B.Cu) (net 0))
 (segment (start 59.944 145.288) (end 68.58 145.288) (width 1) (layer B.Cu) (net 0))
 (segment (start 49.784 145.288) (end 59.944 145.288) (width 1) (layer B.Cu) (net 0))
 (segment (start 30.734 145.288) (end 49.784 145.288) (width 1) (layer B.Cu) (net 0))
 (segment (start 146.304 145.796) (end 149.86 145.796) (width 2) (layer F.Cu) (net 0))
 (segment (start 150.814 144.842) (end 150.814 140.208) (width 2) (layer F.Cu) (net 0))
 (segment (start 149.86 145.796) (end 150.814 144.842) (width 2) (layer F.Cu) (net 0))
 (segment (start 145.734 140.208) (end 144.734 140.208) (width 0.25) (layer F.Cu) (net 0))
 (segment (start 146.304 145.796) (end 131.826 145.796) (width 2) (layer F.Cu) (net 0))
 (segment (start 110.49 145.288) (end 111.814 143.964) (width 1) (layer B.Cu) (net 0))
 (segment (start 33.02 118.364) (end 33.02 147.574) (width 0.25) (layer F.Cu) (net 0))
 (segment (start 36.322 118.11) (end 33.274 118.11) (width 0.25) (layer F.Cu) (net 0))
 (segment (start 33.274 118.11) (end 33.02 118.364) (width 0.25) (layer F.Cu) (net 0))
 (segment (start 104.902 147.574) (end 114.808 147.574) (width 0.25) (layer F.Cu) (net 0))
 (segment (start 104.902 147.574) (end 105.41 147.574) (width 0.25) (layer F.Cu) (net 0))
 (segment (start 33.02 147.574) (end 104.902 147.574) (width 0.25) (layer F.Cu) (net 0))
 (segment (start 114.808 147.574) (end 116.894 145.488) (width 0.25) (layer F.Cu) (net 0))
 (segment (start 105.41 146.812) (end 34.544 146.812) (width 0.25) (layer F.Cu) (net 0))
 (segment (start 138.224 133.048) (end 137.668 133.604) (width 0.25) (layer F.Cu) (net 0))
 (segment (start 150.952 119.048) (end 151 119) (width 0.25) (layer F.Cu) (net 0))
 (segment (start 150.952 133.048) (end 150.952 119.048) (width 2) (layer F.Cu) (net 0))
 (segment (start 160.734 133.048) (end 150.952 133.048) (width 2) (layer F.Cu) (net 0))
 (segment (start 150.952 133.048) (end 138.224 133.048) (width 2) (layer F.Cu) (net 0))
 (segment (start 151 75.46) (end 150.54 75) (width 0.25) (layer B.Cu) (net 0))
 (segment (start 68 71) (end 68 79) (width 1) (layer B.Cu) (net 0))
 (segment (start 77.694 71.306) (end 78 71) (width 0.25) (layer B.Cu) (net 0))
 (segment (start 77.694 91.694) (end 77.694 71.306) (width 1) (layer B.Cu) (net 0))
 (segment (start 78 71) (end 68 71) (width 1) (layer B.Cu) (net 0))
 (segment (start 72.898 91.694) (end 77.694 91.694) (width 1) (layer B.Cu) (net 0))
 (segment (start 77.694 91.694) (end 82.898 91.694) (width 1) (layer B.Cu) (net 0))
 (segment (start 106.73 71.27) (end 107 71) (width 1) (layer B.Cu) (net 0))
 (segment (start 106.73 80.772) (end 106.73 71.27) (width 1) (layer B.Cu) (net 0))
 (segment (start 107 71) (end 78 71) (width 1) (layer B.Cu) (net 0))
 (segment (start 113.95 72.05) (end 115 71) (width 1) (layer B.Cu) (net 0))
 (segment (start 113.95 80.772) (end 113.95 72.05) (width 1) (layer B.Cu) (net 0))
 (segment (start 115 71) (end 107 71) (width 1) (layer B.Cu) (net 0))
 (segment (start 56.062 123.19) (end 55.626 123.626) (width 0.25) (layer F.Cu) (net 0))
 (segment (start 61.322 123.19) (end 56.062 123.19) (width 1) (layer F.Cu) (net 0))
 (segment (start 55.626 123.626) (end 55.626 131.826) (width 1) (layer F.Cu) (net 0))
 (segment (start 55.626 110.998) (end 55.626 123.626) (width 1) (layer F.Cu) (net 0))
 (segment (start 61.322 123.19) (end 73.81 123.19) (width 1) (layer F.Cu) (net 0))
 (segment (start 73.81 123.19) (end 76 121) (width 1) (layer F.Cu) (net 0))
 (segment (start 76 92.256) (end 72.898 89.154) (width 1) (layer F.Cu) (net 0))
 (segment (start 76 121) (end 76 92.256) (width 1) (layer F.Cu) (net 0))
 (segment (start 158.6 91) (end 158.6 80.52) (width 1) (layer F.Cu) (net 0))
 (segment (start 61.322 71.678) (end 61.322 77.47) (width 1) (layer F.Cu) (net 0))
 (segment (start 63 70) (end 61.322 71.678) (width 1) (layer F.Cu) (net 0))
 (segment (start 101.65 89.35) (end 101.65 80.772) (width 0.25) (layer F.Cu) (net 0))
 (segment (start 96.766 94.234) (end 101.65 89.35) (width 0.25) (layer F.Cu) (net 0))
 (segment (start 82.898 94.234) (end 96.766 94.234) (width 0.25) (layer F.Cu) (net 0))
 (segment (start 82.898 96.774) (end 98.774 96.774) (width 0.25) (layer F.Cu) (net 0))
 (segment (start 98.774 96.774) (end 104 91.548) (width 0.25) (layer F.Cu) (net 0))
 (segment (start 104 80.962) (end 104.19 80.772) (width 0.25) (layer F.Cu) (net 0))
 (segment (start 104 91.548) (end 104 80.962) (width 0.25) (layer F.Cu) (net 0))
 (segment (start 87 75) (end 85 77) (width 1) (layer F.Cu) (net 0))
 (segment (start 85 77) (end 85 89) (width 1) (layer F.Cu) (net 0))
 (segment (start 83.052 89) (end 82.898 89.154) (width 0.25) (layer F.Cu) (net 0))
 (segment (start 85 89) (end 83.052 89) (width 1) (layer F.Cu) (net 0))
 (segment (start 100 75) (end 87 75) (width 1) (layer F.Cu) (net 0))
 (segment (start 121 75) (end 121 78.802) (width 1) (layer F.Cu) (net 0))
 (segment (start 121 78.802) (end 119.03 80.772) (width 1) (layer F.Cu) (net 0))
 (segment (start 121 75) (end 100 75) (width 1) (layer F.Cu) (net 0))
 (segment (start 165.814 119.386) (end 166.2 119) (width 0.25) (layer F.Cu) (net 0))
 (segment (start 138.224 133.048) (end 128.952 133.048) (width 2) (layer F.Cu) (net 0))
 (segment (start 128.952 133.048) (end 126 136) (width 2) (layer F.Cu) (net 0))
 (segment (start 126 139.942) (end 125.734 140.208) (width 0.25) (layer F.Cu) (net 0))
 (segment (start 165.814 119.386) (end 166.2 119) (width 0.25) (layer B.Cu) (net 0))
 (segment (start 165.814 140.208) (end 165.814 119.386) (width 2) (layer B.Cu) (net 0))
 (segment (start 139 109) (end 137 111) (width 2) (layer B.Cu) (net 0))
 (segment (start 164 109) (end 139 109) (width 2) (layer B.Cu) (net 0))
 (segment (start 137 111) (end 137 115.92) (width 2) (layer B.Cu) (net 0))
 (segment (start 166.2 111.2) (end 164 109) (width 2) (layer B.Cu) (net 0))
 (segment (start 166.2 119) (end 166.2 111.2) (width 2) (layer B.Cu) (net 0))
 (segment (start 137 115.92) (end 137 121) (width 2) (layer B.Cu) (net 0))
 (segment (start 99.11 75.89) (end 100 75) (width 1) (layer F.Cu) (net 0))
 (segment (start 99.11 80.772) (end 99.11 75.89) (width 1) (layer F.Cu) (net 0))
 (segment (start 158.52 80.52) (end 153 75) (width 1) (layer F.Cu) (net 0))
 (segment (start 158.6 80.52) (end 158.52 80.52) (width 0.25) (layer F.Cu) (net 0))
 (segment (start 153 75) (end 153 72) (width 1) (layer F.Cu) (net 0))
 (segment (start 153 72) (end 151 70) (width 1) (layer F.Cu) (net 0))
 (segment (start 151 70) (end 87 70) (width 1) (layer F.Cu) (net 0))
 (segment (start 87 70) (end 63 70) (width 1) (layer F.Cu) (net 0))
 (segment (start 88 70) (end 87 70) (width 1) (layer F.Cu) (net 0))
 (segment (start 147.92 75) (end 121 75) (width 1) (layer F.Cu) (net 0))
 (segment (start 151 75.54) (end 150.46 75) (width 0.25) (layer B.Cu) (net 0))
 (segment (start 151 91) (end 151 75.54) (width 1) (layer B.Cu) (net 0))
 (segment (start 150.46 75) (end 150.46 73.46) (width 0.25) (layer B.Cu) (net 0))
 (segment (start 148 71) (end 115 71) (width 1) (layer B.Cu) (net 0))
 (segment (start 150.46 73.46) (end 148 71) (width 1) (layer B.Cu) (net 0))
 (segment (start 78.894 132.488) (end 78.74 132.334) (width 0.25) (layer F.Cu) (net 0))
 (segment (start 78.894 142.208) (end 78.894 132.488) (width 1) (layer F.Cu) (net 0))
 (segment (start 97.894 142.208) (end 97.894 132.692) (width 1) (layer F.Cu) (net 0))
 (segment (start 49.734 145.238) (end 49.784 145.288) (width 0.25) (layer B.Cu) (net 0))
 (segment (start 49.734 142.208) (end 49.734 145.238) (width 1) (layer B.Cu) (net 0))
 (segment (start 68.734 145.134) (end 68.58 145.288) (width 0.25) (layer B.Cu) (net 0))
 (segment (start 68.734 142.208) (end 68.734 145.134) (width 1) (layer B.Cu) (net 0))
 (segment (start 87.734 145.138) (end 87.884 145.288) (width 0.25) (layer B.Cu) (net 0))
 (segment (start 87.734 142.208) (end 87.734 145.138) (width 1) (layer B.Cu) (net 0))
 (segment (start 97.79 145.288) (end 110.49 145.288) (width 1) (layer B.Cu) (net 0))
 (segment (start 59.894 132.538) (end 59.69 132.334) (width 0.25) (layer F.Cu) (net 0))
 (segment (start 59.894 142.208) (end 59.894 132.538) (width 1) (layer F.Cu) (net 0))
 (segment (start 40.894 142.208) (end 40.894 132.588) (width 1) (layer F.Cu) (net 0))
 (segment (start 92.71 142.312) (end 92.814 142.208) (width 0.25) (layer F.Cu) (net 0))
 (segment (start 92.71 146.05) (end 92.71 142.312) (width 0.25) (layer F.Cu) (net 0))
 (segment (start 73.914 142.308) (end 73.814 142.208) (width 0.25) (layer F.Cu) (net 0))
 (segment (start 73.914 146.05) (end 73.914 142.308) (width 0.25) (layer F.Cu) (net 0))
 (segment (start 54.95 142.344) (end 54.814 142.208) (width 0.25) (layer F.Cu) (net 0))
 (segment (start 54.95 146.05) (end 54.95 142.344) (width 0.25) (layer F.Cu) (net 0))
 (segment (start 54.864 146.05) (end 54.95 146.05) (width 0.25) (layer F.Cu) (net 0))
 (segment (start 54.95 146.05) (end 73.914 146.05) (width 0.25) (layer F.Cu) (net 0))
 (segment (start 105.41 143.532) (end 106.734 142.208) (width 0.25) (layer F.Cu) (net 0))
 (segment (start 105.41 146.812) (end 105.41 143.532) (width 0.25) (layer F.Cu) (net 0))
 (segment (start 116.894 145.488) (end 116.894 142.208) (width 0.25) (layer F.Cu) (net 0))
 (segment (start 111.814 142.208) (end 111.814 143.964) (width 1) (layer B.Cu) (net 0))
 (segment (start 131.826 145.796) (end 131.796 145.796) (width 0.25) (layer F.Cu) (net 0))
 (segment (start 130.814 144.814) (end 130.814 142.208) (width 2) (layer F.Cu) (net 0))
 (segment (start 131.796 145.796) (end 130.814 144.814) (width 2) (layer F.Cu) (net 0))
 (segment (start 125.734 136.266) (end 126 136) (width 0.25) (layer F.Cu) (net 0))
 (segment (start 125.734 142.208) (end 125.734 136.266) (width 2) (layer F.Cu) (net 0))
 (segment (start 135.894 142.208) (end 135.894 141.106) (width 2) (layer F.Cu) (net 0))
 (segment (start 136.792 140.208) (end 145.734 140.208) (width 2) (layer F.Cu) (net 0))
 (segment (start 135.894 141.106) (end 136.792 140.208) (width 2) (layer F.Cu) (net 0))
 (segment (start 34.544 146.812) (end 34.544 145.544) (width 0.25) (layer F.Cu) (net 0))
 (segment (start 34.544 145.544) (end 34 145) (width 0.25) (layer F.Cu) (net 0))
 (segment (start 34 122.972) (end 36.322 120.65) (width 0.25) (layer F.Cu) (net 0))
 (segment (start 34 145) (end 34 122.972) (width 0.25) (layer F.Cu) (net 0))
 (segment (start 61.322 90.17) (end 66.04 90.17) (width 1) (layer B.Cu) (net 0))
 (segment (start 68 88.21) (end 68 79) (width 1) (layer B.Cu) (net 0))
 (segment (start 66.04 90.17) (end 68 88.21) (width 1) (layer B.Cu) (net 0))
 (segment (start 31.75 115.57) (end 30.48 114.3) (width 0.25) (layer F.Cu) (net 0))
 (segment (start 36.322 115.57) (end 31.75 115.57) (width 0.25) (layer F.Cu) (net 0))
 (segment (start 36.322 113.03) (end 34.29 113.03) (width 0.25) (layer F.Cu) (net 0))
 (segment (start 34.29 113.03) (end 33.02 111.76) (width 0.25) (layer F.Cu) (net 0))
 (segment (start 33.02 111.76) (end 30.48 111.76) (width 0.25) (layer F.Cu) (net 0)))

